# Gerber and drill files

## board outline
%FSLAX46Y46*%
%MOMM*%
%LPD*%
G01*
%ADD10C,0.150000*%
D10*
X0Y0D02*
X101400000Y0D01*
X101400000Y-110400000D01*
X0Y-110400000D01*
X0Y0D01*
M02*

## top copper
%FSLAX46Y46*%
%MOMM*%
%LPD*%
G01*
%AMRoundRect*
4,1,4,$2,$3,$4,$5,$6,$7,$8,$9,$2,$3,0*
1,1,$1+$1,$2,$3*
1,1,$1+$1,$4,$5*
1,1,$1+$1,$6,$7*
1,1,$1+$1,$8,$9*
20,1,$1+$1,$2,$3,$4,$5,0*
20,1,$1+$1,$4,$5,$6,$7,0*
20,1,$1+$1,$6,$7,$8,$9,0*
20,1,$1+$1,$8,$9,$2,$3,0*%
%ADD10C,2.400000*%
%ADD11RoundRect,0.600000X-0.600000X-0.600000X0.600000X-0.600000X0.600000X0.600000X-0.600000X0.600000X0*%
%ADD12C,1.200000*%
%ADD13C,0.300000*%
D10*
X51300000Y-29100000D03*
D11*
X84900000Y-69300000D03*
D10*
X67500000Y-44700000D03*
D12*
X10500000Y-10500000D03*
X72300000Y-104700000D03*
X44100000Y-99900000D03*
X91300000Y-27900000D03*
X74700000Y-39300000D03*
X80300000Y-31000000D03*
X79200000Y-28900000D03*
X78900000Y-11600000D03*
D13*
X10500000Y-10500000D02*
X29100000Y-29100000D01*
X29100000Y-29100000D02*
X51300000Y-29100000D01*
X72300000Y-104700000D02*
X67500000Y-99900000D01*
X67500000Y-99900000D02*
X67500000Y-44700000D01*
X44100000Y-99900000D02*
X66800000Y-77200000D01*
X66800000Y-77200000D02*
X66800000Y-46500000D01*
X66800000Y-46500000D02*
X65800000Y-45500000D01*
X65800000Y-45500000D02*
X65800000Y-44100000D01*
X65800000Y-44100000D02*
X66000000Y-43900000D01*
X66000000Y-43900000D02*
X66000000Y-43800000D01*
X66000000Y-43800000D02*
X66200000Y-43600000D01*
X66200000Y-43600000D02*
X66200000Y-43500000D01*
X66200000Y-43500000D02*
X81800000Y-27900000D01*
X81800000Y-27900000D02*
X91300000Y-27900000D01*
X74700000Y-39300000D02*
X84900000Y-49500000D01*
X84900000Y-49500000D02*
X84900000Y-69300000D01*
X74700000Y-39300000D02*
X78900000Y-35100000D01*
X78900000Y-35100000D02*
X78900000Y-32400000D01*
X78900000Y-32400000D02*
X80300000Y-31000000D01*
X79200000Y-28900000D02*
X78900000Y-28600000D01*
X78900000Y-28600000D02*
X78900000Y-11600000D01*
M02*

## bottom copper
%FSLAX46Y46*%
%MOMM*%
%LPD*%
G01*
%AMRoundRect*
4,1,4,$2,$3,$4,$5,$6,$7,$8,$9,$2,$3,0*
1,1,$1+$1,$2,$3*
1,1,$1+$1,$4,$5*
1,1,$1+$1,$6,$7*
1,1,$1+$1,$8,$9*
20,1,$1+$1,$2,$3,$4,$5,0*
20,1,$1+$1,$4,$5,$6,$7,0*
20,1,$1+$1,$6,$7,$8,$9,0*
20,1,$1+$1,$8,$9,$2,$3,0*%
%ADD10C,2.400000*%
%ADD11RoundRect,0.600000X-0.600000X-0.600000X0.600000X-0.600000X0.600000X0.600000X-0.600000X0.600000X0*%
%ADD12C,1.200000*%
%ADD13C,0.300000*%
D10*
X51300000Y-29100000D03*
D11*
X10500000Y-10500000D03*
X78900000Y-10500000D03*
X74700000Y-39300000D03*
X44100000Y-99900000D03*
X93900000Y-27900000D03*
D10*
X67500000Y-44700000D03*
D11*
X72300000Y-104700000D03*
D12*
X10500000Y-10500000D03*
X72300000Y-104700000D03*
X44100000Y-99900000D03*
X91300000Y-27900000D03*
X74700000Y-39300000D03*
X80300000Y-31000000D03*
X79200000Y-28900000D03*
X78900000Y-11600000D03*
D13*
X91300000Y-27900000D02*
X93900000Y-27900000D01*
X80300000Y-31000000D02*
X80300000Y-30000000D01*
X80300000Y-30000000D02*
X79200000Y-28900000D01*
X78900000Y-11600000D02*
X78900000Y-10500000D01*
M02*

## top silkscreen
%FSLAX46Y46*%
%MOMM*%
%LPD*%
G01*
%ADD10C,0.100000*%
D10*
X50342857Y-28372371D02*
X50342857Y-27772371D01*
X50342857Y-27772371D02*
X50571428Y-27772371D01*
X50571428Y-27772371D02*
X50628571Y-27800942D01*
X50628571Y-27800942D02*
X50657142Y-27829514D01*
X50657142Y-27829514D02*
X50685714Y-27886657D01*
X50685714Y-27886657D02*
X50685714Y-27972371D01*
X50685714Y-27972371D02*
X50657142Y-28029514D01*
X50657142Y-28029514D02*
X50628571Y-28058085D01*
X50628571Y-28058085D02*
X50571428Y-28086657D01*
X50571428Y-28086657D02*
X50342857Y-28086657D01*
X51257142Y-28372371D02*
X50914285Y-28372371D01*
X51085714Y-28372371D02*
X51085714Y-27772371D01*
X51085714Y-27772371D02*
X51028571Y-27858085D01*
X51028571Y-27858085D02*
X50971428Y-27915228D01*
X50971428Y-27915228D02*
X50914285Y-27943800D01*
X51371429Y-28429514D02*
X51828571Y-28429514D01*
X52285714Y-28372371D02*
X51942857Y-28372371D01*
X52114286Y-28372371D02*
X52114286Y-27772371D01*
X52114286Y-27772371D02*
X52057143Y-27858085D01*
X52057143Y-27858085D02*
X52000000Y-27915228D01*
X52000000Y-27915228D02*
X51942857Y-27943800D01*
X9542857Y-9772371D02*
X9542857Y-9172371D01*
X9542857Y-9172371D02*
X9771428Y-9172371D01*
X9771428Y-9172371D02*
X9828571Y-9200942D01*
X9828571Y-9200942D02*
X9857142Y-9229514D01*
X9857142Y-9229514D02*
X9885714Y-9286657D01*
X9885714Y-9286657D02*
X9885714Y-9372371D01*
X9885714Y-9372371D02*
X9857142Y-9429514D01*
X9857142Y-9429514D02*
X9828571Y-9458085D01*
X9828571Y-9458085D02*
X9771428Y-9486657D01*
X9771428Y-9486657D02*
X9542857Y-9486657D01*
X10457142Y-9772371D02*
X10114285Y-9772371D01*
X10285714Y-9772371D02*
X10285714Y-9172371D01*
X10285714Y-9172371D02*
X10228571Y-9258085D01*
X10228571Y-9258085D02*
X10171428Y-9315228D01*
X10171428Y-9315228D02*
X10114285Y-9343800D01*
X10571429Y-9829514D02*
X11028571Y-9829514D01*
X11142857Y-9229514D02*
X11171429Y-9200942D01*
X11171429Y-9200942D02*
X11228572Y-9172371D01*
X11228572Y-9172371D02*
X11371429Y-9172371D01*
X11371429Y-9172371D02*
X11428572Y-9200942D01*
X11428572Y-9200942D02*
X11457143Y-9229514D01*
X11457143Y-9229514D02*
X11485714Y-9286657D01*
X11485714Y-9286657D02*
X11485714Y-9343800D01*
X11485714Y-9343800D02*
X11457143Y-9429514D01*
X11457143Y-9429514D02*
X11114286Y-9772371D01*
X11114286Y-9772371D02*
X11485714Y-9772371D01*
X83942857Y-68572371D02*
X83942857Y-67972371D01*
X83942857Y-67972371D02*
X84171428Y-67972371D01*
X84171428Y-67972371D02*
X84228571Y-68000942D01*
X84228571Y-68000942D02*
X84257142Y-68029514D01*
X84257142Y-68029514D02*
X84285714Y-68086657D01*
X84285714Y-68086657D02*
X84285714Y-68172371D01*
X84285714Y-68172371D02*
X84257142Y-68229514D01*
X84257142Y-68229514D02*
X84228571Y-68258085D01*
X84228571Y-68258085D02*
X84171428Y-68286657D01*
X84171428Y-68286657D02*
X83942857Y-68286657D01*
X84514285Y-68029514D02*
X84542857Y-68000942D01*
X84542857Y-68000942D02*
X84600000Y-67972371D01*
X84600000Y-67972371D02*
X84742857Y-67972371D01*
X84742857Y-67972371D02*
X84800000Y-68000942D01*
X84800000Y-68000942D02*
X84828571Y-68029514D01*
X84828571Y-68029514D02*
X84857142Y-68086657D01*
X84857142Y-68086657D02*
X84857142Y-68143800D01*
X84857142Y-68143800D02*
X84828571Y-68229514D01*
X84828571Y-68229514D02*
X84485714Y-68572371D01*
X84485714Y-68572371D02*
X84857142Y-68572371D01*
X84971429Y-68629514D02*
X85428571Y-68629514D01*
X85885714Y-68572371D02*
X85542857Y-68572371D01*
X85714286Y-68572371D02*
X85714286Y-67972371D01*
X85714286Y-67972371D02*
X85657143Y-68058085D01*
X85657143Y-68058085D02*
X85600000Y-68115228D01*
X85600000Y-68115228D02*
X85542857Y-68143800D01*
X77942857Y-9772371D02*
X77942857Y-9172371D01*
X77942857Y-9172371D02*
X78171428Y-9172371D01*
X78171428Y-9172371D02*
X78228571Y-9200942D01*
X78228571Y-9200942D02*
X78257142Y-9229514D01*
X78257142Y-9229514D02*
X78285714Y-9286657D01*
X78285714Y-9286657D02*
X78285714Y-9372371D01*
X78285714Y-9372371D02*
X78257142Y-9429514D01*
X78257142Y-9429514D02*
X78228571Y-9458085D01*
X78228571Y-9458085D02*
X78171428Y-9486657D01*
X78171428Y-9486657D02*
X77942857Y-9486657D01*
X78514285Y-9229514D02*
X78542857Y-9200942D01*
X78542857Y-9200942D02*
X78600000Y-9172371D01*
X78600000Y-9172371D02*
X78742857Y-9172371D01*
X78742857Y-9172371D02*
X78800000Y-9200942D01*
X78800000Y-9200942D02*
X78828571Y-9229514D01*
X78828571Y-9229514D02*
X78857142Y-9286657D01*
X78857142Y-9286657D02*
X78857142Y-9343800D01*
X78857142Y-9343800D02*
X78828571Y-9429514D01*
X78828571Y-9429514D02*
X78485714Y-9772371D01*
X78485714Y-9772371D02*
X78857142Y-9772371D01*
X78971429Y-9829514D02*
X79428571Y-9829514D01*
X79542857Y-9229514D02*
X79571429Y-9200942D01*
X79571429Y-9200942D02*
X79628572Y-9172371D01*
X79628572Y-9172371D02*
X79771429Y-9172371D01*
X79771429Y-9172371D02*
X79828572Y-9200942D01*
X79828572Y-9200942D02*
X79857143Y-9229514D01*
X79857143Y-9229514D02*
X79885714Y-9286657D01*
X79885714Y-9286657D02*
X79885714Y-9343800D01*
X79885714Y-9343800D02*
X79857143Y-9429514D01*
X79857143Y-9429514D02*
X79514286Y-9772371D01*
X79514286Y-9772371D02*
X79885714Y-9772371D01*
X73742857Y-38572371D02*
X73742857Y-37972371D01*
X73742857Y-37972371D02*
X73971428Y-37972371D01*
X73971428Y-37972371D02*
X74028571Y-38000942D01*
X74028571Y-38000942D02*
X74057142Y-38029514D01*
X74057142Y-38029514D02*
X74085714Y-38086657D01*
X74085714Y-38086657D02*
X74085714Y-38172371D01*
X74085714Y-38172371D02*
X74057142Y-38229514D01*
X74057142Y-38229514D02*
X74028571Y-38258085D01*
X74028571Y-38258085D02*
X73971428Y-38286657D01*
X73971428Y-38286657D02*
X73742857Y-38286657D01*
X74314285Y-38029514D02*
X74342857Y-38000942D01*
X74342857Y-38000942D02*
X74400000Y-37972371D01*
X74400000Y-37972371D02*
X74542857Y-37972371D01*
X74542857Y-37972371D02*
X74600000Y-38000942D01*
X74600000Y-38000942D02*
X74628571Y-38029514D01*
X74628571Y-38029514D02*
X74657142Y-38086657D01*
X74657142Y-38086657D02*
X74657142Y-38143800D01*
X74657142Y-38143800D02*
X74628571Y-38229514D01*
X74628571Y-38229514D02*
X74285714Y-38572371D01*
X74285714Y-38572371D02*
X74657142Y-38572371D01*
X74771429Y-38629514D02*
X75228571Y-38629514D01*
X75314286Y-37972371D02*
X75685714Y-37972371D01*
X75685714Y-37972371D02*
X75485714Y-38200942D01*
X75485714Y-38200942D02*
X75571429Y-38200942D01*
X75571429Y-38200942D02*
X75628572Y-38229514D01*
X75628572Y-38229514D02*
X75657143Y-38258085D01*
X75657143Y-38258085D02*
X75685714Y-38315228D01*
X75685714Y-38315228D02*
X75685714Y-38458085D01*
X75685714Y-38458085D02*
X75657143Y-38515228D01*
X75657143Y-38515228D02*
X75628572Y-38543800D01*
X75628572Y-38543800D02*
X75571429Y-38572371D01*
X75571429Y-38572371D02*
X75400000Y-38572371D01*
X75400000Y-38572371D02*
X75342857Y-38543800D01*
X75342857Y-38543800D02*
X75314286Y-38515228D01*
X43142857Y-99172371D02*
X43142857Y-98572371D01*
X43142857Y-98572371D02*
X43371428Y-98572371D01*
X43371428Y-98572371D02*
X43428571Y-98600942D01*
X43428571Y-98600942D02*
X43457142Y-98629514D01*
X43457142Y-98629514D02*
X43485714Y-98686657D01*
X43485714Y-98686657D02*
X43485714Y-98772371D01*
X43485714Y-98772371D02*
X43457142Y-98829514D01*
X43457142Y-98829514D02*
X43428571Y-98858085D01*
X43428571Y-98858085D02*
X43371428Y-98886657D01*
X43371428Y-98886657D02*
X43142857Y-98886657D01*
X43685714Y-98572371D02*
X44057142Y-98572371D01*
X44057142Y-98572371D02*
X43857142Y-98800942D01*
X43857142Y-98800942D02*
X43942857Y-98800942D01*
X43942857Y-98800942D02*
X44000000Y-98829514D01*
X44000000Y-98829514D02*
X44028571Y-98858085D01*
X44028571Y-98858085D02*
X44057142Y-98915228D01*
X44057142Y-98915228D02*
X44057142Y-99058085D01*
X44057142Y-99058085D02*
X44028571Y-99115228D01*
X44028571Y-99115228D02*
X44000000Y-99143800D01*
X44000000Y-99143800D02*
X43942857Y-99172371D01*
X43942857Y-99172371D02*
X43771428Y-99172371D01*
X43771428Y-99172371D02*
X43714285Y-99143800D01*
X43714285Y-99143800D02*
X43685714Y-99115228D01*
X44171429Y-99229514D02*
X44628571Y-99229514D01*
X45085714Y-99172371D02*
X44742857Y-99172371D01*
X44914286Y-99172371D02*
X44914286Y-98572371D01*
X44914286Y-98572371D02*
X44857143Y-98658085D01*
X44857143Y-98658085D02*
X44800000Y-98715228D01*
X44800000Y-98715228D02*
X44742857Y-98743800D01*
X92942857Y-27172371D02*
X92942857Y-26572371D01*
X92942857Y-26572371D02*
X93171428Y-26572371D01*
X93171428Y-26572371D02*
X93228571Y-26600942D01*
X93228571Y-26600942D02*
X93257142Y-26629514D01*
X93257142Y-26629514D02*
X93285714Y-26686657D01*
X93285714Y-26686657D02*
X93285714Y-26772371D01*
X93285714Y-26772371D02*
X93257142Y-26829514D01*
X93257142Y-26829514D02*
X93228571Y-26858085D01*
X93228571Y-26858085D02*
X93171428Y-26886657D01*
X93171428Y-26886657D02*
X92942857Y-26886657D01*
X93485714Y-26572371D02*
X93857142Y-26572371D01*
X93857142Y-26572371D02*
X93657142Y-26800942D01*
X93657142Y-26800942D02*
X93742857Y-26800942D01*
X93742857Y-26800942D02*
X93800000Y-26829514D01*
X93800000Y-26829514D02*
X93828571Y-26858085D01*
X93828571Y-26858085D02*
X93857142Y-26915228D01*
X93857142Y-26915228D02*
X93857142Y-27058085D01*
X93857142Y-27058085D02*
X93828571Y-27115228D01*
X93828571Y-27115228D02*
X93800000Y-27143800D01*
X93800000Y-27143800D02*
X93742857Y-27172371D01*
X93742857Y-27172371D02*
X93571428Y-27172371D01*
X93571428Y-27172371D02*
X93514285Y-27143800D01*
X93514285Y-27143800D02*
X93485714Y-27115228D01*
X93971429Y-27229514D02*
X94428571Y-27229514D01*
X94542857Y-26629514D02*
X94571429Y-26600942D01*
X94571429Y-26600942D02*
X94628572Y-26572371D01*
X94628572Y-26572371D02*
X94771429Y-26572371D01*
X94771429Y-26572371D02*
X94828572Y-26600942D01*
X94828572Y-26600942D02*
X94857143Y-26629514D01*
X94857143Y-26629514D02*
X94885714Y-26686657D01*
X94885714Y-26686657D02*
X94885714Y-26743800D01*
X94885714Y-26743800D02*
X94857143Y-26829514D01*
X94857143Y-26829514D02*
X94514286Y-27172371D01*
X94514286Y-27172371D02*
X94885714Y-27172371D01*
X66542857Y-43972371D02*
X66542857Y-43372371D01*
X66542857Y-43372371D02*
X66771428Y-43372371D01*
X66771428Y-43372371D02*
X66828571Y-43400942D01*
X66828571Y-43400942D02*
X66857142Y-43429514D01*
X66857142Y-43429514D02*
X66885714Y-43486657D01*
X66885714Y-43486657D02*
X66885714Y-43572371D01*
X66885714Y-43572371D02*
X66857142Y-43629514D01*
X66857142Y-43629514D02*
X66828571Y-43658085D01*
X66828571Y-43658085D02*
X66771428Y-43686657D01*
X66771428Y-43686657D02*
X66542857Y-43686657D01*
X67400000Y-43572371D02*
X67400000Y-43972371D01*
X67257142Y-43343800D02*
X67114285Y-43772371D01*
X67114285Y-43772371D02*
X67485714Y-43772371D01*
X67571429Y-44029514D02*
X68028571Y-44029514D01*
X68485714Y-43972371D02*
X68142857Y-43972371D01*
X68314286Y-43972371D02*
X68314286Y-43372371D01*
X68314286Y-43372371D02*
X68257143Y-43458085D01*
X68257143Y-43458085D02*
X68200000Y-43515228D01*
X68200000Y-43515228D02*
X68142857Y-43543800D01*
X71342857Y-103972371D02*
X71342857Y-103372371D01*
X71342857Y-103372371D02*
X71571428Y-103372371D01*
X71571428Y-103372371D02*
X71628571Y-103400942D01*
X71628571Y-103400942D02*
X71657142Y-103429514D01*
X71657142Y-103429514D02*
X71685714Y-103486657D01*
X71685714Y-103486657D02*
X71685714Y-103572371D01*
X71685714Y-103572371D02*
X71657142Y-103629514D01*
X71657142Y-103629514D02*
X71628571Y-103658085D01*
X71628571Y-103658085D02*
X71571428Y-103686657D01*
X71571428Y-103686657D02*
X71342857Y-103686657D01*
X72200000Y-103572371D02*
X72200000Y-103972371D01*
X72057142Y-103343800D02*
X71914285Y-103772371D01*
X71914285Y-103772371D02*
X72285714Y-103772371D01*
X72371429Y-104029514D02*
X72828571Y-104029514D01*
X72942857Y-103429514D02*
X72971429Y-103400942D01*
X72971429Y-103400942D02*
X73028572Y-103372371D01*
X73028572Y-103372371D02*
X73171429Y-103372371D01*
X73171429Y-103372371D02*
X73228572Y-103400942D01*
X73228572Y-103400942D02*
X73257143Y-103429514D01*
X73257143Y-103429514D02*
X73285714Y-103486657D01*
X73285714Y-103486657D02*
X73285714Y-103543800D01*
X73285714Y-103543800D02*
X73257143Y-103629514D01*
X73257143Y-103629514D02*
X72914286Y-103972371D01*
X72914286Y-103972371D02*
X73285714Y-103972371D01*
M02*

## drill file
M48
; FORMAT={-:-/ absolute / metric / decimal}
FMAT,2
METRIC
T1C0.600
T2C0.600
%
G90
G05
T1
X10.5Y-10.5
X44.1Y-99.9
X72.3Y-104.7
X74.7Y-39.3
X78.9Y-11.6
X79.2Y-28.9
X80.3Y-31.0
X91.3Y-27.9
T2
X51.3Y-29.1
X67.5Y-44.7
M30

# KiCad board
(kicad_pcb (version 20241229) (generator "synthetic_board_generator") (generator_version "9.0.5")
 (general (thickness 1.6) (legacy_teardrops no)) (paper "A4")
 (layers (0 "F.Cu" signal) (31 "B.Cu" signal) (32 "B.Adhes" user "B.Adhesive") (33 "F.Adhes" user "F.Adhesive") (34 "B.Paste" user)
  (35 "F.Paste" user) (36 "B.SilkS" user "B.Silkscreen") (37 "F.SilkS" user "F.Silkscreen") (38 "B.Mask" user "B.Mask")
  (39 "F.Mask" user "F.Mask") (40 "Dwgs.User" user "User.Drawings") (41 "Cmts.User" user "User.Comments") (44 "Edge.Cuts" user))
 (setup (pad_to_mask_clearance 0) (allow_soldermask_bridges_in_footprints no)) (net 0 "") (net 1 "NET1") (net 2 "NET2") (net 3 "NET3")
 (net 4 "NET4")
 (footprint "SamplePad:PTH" (layer "F.Cu") (at 51.300000 29.100000)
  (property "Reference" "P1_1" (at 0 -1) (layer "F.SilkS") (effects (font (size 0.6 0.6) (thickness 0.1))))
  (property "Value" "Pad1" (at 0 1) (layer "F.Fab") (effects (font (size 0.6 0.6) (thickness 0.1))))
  (pad "1" thru_hole circle (at 0 0) (size 2.4 2.4) (drill 0.6) (layers "*.Cu" "*.Mask") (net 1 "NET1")))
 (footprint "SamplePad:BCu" (layer "B.Cu") (at 10.500000 10.500000)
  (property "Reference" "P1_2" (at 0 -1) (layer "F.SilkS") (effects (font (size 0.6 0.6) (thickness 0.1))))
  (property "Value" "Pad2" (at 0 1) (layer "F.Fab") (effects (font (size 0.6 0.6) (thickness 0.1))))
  (pad "1" smd roundrect (at 0 0) (size 2.4 2.4) (layers "B.Cu" "B.Paste" "B.Mask") (roundrect_rratio 0.25) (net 1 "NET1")))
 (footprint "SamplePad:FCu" (layer "F.Cu") (at 84.900000 69.300000)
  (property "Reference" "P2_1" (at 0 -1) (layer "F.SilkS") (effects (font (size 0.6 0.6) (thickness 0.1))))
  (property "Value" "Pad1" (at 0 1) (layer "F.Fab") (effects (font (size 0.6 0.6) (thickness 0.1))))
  (pad "1" smd roundrect (at 0 0) (size 2.4 2.4) (layers "F.Cu" "F.Paste" "F.Mask") (roundrect_rratio 0.25) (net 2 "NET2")))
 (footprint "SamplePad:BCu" (layer "B.Cu") (at 78.900000 10.500000)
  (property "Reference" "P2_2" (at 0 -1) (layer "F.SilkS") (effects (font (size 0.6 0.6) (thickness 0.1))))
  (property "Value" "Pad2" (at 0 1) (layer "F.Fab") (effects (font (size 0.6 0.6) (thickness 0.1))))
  (pad "1" smd roundrect (at 0 0) (size 2.4 2.4) (layers "B.Cu" "B.Paste" "B.Mask") (roundrect_rratio 0.25) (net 2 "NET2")))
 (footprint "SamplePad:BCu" (layer "B.Cu") (at 74.700000 39.300000)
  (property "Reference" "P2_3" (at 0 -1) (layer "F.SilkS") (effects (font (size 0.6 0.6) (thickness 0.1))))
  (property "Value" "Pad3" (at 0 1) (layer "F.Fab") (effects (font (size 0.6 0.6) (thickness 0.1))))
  (pad "1" smd roundrect (at 0 0) (size 2.4 2.4) (layers "B.Cu" "B.Paste" "B.Mask") (roundrect_rratio 0.25) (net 2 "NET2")))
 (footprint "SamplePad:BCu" (layer "B.Cu") (at 44.100000 99.900000)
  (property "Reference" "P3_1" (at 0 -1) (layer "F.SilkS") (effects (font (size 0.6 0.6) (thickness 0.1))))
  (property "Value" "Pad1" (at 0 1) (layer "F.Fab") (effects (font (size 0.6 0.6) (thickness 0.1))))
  (pad "1" smd roundrect (at 0 0) (size 2.4 2.4) (layers "B.Cu" "B.Paste" "B.Mask") (roundrect_rratio 0.25) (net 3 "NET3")))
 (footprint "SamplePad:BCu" (layer "B.Cu") (at 93.900000 27.900000)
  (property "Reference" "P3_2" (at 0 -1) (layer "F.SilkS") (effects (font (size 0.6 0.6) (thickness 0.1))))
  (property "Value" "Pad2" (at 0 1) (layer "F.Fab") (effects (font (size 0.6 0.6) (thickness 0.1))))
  (pad "1" smd roundrect (at 0 0) (size 2.4 2.4) (layers "B.Cu" "B.Paste" "B.Mask") (roundrect_rratio 0.25) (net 3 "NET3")))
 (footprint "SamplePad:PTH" (layer "F.Cu") (at 67.500000 44.700000)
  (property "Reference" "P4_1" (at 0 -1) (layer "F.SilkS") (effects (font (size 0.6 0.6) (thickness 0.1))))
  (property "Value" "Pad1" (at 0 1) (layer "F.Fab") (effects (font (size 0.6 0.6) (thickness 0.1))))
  (pad "1" thru_hole circle (at 0 0) (size 2.4 2.4) (drill 0.6) (layers "*.Cu" "*.Mask") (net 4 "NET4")))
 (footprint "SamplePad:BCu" (layer "B.Cu") (at 72.300000 104.700000)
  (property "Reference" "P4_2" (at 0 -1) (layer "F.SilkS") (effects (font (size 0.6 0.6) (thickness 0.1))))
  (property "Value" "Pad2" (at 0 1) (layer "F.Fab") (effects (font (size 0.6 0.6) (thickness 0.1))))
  (pad "1" smd roundrect (at 0 0) (size 2.4 2.4) (layers "B.Cu" "B.Paste" "B.Mask") (roundrect_rratio 0.25) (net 4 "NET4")))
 (gr_rect (start 0.0 0.0) (end 101.4 110.4) (stroke (width 0.15) (type solid)) (fill none) (layer "Edge.Cuts"))
 (segment (start 10.500000 10.500000) (end 29.100000 29.100000) (width 0.3) (layer "F.Cu") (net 1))
 (segment (start 29.100000 29.100000) (end 51.300000 29.100000) (width 0.3) (layer "F.Cu") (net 1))
 (via (at 10.500000 10.500000) (size 1.2) (drill 0.6) (layers "F.Cu" "B.Cu") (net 1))
 (segment (start 72.300000 104.700000) (end 67.500000 99.900000) (width 0.3) (layer "F.Cu") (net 4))
 (segment (start 67.500000 99.900000) (end 67.500000 44.700000) (width 0.3) (layer "F.Cu") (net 4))
 (via (at 72.300000 104.700000) (size 1.2) (drill 0.6) (layers "F.Cu" "B.Cu") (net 4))
 (segment (start 44.100000 99.900000) (end 66.800000 77.200000) (width 0.3) (layer "F.Cu") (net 3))
 (segment (start 66.800000 77.200000) (end 66.800000 46.500000) (width 0.3) (layer "F.Cu") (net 3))
 (segment (start 66.800000 46.500000) (end 65.800000 45.500000) (width 0.3) (layer "F.Cu") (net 3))
 (segment (start 65.800000 45.500000) (end 65.800000 44.100000) (width 0.3) (layer "F.Cu") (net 3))
 (segment (start 65.800000 44.100000) (end 66.000000 43.900000) (width 0.3) (layer "F.Cu") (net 3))
 (segment (start 66.000000 43.900000) (end 66.000000 43.800000) (width 0.3) (layer "F.Cu") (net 3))
 (segment (start 66.000000 43.800000) (end 66.200000 43.600000) (width 0.3) (layer "F.Cu") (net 3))
 (segment (start 66.200000 43.600000) (end 66.200000 43.500000) (width 0.3) (layer "F.Cu") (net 3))
 (segment (start 66.200000 43.500000) (end 81.800000 27.900000) (width 0.3) (layer "F.Cu") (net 3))
 (segment (start 81.800000 27.900000) (end 91.300000 27.900000) (width 0.3) (layer "F.Cu") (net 3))
 (segment (start 91.300000 27.900000) (end 93.900000 27.900000) (width 0.3) (layer "B.Cu") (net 3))
 (via (at 44.100000 99.900000) (size 1.2) (drill 0.6) (layers "F.Cu" "B.Cu") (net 3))
 (via (at 91.300000 27.900000) (size 1.2) (drill 0.6) (layers "F.Cu" "B.Cu") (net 3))
 (segment (start 74.700000 39.300000) (end 84.900000 49.500000) (width 0.3) (layer "F.Cu") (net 2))
 (segment (start 84.900000 49.500000) (end 84.900000 69.300000) (width 0.3) (layer "F.Cu") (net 2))
 (segment (start 74.700000 39.300000) (end 78.900000 35.100000) (width 0.3) (layer "F.Cu") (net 2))
 (segment (start 78.900000 35.100000) (end 78.900000 32.400000) (width 0.3) (layer "F.Cu") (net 2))
 (segment (start 78.900000 32.400000) (end 80.300000 31.000000) (width 0.3) (layer "F.Cu") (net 2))
 (segment (start 79.200000 28.900000) (end 78.900000 28.600000) (width 0.3) (layer "F.Cu") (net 2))
 (segment (start 78.900000 28.600000) (end 78.900000 11.600000) (width 0.3) (layer "F.Cu") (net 2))
 (segment (start 80.300000 31.000000) (end 80.300000 30.000000) (width 0.3) (layer "B.Cu") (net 2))
 (segment (start 80.300000 30.000000) (end 79.200000 28.900000) (width 0.3) (layer "B.Cu") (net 2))
 (segment (start 78.900000 11.600000) (end 78.900000 10.500000) (width 0.3) (layer "B.Cu") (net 2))
 (via (at 74.700000 39.300000) (size 1.2) (drill 0.6) (layers "F.Cu" "B.Cu") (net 2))
 (via (at 80.300000 31.000000) (size 1.2) (drill 0.6) (layers "F.Cu" "B.Cu") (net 2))
 (via (at 79.200000 28.900000) (size 1.2) (drill 0.6) (layers "F.Cu" "B.Cu") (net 2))
 (via (at 78.900000 11.600000) (size 1.2) (drill 0.6) (layers "F.Cu" "B.Cu") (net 2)))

